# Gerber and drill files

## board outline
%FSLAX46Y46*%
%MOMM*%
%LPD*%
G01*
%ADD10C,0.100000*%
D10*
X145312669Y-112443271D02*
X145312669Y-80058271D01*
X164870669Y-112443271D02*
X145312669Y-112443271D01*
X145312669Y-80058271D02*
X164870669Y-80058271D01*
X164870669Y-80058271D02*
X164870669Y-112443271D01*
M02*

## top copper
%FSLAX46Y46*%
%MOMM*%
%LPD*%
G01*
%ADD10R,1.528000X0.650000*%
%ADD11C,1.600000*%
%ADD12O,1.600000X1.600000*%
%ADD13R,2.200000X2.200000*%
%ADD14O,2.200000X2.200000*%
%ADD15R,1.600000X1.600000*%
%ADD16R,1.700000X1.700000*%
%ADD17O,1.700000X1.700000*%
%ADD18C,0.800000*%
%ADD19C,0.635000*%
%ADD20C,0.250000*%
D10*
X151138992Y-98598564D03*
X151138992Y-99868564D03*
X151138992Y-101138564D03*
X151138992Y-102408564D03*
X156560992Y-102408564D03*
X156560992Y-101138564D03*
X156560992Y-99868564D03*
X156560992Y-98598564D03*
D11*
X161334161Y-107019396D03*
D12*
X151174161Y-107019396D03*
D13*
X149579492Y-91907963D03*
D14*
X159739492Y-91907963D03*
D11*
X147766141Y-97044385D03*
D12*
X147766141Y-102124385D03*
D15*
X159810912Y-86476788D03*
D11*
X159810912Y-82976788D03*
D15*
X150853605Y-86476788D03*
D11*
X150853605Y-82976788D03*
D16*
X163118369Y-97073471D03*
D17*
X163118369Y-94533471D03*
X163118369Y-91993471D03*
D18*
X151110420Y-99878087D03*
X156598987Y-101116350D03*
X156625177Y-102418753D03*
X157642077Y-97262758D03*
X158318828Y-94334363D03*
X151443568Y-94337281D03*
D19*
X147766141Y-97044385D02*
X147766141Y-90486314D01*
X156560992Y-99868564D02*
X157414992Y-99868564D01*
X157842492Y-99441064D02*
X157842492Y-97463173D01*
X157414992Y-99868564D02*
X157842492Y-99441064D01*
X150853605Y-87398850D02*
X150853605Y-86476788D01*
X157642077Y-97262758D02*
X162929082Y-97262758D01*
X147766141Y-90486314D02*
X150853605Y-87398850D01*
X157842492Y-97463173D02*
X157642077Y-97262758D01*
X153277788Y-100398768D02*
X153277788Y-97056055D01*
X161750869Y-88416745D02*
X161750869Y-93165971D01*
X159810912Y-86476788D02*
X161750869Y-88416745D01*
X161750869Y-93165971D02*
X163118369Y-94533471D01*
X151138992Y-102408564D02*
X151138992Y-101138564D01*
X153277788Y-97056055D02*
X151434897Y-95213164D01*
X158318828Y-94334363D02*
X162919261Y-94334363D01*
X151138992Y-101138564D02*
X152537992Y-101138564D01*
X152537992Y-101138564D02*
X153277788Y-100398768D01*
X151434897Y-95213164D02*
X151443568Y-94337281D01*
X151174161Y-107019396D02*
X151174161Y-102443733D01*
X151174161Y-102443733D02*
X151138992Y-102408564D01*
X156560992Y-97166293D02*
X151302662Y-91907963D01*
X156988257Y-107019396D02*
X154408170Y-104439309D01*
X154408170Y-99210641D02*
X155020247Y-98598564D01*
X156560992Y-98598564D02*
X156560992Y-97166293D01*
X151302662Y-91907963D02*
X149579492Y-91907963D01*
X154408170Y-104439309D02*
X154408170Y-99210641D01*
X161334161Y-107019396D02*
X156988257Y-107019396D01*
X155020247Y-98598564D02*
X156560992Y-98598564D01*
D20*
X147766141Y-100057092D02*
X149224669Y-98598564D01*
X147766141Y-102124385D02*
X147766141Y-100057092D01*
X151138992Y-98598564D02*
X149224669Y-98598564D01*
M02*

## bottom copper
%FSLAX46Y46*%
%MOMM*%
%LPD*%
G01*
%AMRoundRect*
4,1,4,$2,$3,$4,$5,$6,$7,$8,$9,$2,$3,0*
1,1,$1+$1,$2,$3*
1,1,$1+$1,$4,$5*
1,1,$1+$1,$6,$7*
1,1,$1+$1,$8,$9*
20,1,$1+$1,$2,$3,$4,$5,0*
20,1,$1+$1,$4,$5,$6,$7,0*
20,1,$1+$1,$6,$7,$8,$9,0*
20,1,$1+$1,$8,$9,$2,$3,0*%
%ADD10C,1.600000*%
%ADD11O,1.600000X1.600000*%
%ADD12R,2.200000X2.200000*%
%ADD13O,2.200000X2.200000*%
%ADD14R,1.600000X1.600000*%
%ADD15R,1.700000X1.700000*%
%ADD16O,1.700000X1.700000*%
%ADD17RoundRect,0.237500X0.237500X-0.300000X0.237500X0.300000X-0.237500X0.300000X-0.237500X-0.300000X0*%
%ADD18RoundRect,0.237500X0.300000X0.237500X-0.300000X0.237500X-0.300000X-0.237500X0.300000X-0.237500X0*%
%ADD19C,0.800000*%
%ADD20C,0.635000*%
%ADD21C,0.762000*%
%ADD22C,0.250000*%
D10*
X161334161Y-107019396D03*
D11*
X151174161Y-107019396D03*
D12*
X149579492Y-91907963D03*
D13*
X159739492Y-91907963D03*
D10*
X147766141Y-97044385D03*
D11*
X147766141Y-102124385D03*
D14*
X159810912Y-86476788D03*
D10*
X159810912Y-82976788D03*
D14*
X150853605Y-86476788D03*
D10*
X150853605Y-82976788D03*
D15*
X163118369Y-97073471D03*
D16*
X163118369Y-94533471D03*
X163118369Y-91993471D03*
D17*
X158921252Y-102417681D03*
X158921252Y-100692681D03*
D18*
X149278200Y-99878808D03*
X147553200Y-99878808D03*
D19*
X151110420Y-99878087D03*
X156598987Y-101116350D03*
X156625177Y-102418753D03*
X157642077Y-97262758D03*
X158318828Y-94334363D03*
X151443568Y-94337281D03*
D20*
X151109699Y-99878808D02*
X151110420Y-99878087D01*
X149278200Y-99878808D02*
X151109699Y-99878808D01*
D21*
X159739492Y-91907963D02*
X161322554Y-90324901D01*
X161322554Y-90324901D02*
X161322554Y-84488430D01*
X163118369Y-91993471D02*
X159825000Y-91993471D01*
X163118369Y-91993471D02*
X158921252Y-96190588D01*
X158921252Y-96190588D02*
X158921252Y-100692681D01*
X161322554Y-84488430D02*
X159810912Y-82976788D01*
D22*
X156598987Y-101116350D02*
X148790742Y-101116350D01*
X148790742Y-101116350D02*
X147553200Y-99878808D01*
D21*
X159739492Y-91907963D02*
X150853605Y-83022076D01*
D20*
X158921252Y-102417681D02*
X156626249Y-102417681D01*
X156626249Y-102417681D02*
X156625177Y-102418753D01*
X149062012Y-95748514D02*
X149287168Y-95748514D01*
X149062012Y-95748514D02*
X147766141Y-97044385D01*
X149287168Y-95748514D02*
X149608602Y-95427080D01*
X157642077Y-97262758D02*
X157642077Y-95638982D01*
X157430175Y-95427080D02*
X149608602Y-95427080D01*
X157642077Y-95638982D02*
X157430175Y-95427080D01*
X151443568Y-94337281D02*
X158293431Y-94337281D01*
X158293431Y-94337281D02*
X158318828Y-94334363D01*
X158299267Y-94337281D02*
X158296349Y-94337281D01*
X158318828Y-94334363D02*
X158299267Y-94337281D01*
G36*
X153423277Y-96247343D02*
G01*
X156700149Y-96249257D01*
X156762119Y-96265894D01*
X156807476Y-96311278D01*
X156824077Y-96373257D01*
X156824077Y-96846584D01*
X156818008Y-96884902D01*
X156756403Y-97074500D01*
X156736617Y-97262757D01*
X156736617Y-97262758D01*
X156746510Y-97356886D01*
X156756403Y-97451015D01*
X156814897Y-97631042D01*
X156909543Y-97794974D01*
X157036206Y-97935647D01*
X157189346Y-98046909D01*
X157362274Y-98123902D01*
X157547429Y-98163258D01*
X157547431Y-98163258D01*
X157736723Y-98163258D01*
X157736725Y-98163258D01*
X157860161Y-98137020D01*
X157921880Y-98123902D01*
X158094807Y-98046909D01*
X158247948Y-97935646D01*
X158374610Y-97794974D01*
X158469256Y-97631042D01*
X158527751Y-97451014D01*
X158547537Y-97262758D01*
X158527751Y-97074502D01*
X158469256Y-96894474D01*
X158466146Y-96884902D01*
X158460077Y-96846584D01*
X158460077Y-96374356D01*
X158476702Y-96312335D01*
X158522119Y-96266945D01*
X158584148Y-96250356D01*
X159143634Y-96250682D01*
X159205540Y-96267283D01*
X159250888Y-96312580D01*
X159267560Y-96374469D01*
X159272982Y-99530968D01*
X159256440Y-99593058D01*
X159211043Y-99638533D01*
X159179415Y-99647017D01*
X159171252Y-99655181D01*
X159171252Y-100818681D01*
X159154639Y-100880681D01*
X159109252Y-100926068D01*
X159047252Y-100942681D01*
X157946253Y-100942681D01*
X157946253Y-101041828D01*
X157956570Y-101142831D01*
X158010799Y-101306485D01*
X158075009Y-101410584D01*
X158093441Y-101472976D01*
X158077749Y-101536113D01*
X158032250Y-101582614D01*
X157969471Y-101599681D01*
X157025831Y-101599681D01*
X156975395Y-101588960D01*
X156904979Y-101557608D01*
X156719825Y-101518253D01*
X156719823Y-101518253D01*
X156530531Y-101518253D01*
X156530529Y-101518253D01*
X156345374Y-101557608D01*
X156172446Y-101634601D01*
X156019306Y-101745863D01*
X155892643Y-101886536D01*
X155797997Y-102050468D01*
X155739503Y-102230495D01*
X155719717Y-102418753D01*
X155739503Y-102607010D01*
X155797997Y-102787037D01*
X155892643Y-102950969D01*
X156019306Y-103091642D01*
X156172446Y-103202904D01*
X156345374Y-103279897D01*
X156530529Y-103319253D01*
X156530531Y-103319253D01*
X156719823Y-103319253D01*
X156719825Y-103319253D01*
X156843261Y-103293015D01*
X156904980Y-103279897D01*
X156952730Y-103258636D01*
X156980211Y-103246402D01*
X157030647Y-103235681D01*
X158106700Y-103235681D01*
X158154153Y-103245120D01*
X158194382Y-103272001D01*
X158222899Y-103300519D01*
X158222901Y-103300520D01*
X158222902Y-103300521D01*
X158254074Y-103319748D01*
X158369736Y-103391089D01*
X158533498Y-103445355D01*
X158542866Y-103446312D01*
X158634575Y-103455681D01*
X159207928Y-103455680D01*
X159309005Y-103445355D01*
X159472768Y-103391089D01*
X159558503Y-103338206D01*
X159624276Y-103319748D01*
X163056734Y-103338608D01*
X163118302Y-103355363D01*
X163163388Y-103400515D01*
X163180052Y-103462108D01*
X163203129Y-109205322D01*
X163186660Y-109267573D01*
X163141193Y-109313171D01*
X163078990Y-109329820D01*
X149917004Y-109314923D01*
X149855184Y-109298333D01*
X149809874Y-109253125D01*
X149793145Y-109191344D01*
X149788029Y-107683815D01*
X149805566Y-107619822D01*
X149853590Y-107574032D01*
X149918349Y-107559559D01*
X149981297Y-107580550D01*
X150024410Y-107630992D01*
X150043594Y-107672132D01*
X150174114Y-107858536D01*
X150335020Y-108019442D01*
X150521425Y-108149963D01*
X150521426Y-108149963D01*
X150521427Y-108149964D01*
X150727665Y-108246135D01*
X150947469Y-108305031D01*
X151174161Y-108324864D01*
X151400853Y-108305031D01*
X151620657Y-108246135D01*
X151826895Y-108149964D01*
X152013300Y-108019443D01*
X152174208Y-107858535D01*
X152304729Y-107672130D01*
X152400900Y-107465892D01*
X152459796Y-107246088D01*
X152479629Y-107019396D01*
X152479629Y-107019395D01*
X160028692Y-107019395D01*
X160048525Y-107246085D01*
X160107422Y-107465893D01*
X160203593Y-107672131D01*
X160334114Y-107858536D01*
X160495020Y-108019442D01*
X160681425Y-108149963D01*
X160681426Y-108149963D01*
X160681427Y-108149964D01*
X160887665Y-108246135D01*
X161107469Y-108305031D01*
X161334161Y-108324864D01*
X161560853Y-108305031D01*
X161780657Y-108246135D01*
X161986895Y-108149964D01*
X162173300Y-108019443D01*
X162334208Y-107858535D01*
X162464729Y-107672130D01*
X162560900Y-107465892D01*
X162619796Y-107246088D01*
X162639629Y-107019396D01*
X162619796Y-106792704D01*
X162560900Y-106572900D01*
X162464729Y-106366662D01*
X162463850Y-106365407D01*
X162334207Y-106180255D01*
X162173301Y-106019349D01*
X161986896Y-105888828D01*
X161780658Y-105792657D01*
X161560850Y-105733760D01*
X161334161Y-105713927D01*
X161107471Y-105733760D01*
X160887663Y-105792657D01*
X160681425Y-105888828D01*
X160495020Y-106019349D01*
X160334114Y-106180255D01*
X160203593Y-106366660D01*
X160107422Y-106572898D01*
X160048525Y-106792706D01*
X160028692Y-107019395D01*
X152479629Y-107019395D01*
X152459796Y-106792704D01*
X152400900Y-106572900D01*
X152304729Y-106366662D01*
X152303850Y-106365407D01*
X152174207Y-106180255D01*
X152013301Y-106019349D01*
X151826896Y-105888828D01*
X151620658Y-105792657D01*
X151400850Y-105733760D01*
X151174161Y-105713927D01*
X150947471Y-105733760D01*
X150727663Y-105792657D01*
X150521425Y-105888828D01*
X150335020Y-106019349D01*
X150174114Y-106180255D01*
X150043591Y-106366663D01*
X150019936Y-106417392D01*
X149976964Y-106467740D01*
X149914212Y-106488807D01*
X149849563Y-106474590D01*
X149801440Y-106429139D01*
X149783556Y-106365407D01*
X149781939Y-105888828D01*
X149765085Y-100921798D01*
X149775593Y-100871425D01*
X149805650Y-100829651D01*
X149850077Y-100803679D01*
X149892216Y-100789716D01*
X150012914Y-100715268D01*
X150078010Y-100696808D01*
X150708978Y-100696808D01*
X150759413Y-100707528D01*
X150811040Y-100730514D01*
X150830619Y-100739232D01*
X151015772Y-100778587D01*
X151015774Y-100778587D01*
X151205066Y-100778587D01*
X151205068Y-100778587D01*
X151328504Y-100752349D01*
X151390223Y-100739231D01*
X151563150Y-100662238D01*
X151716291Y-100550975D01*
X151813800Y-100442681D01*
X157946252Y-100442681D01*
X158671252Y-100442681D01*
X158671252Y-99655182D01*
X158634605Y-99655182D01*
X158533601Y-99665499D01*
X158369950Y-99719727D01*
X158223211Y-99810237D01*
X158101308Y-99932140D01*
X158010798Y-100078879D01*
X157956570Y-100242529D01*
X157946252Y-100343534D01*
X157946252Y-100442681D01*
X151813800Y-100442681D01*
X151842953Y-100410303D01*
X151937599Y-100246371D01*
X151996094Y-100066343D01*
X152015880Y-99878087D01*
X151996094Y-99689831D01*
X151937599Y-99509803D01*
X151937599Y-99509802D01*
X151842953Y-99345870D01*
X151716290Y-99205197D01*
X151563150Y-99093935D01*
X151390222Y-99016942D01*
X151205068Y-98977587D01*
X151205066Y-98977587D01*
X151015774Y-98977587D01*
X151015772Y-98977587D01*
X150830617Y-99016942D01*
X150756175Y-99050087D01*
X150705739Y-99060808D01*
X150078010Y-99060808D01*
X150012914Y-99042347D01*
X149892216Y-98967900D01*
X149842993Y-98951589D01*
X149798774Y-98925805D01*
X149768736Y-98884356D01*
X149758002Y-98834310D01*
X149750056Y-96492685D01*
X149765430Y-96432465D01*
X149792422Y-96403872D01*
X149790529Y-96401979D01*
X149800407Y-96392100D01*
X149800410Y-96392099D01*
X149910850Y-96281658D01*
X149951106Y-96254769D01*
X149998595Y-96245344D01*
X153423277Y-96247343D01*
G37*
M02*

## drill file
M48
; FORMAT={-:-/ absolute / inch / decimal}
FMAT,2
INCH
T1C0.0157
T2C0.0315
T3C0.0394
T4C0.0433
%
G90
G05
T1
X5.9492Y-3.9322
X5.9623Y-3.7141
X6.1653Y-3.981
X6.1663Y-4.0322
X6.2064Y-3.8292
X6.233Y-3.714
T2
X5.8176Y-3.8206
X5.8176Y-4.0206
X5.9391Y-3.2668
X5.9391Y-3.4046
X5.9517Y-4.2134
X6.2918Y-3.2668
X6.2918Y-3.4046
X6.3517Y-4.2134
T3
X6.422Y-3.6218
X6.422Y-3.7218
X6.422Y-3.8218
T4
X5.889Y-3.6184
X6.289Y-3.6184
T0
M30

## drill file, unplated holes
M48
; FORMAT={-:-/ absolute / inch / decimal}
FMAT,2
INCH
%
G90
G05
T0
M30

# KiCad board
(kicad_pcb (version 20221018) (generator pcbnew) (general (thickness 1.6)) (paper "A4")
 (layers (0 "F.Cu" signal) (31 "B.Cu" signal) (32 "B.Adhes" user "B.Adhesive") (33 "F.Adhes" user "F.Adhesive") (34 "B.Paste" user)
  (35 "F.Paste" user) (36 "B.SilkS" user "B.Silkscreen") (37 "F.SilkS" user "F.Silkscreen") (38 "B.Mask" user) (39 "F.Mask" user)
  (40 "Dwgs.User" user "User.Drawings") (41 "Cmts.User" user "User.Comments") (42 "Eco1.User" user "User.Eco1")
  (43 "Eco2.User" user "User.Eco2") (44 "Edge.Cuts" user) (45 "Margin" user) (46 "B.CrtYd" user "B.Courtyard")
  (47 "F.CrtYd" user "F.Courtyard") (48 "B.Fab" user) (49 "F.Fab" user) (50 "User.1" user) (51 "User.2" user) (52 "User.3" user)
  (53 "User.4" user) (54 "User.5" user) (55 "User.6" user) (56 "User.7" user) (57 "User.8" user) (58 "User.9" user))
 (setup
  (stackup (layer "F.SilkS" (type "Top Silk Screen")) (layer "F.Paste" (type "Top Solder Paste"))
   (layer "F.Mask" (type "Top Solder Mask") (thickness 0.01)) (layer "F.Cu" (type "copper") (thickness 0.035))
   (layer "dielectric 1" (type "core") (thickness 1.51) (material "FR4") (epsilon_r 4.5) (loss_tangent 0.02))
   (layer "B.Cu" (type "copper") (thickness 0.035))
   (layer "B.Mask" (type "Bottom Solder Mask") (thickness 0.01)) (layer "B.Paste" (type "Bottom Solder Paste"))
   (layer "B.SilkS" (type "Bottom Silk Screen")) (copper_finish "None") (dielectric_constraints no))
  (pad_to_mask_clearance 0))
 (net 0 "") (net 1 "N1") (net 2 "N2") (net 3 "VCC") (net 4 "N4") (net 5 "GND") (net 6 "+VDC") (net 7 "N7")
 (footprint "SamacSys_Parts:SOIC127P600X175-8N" (layer "F.Cu") (at 153.849992 100.503564)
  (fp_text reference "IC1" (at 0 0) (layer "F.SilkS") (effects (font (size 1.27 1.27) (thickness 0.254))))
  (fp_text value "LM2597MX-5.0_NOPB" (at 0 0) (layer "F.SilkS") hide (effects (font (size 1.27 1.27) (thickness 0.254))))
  (pad "1" smd rect (at -2.711 -1.905 90) (size 0.65 1.528) (layers "F.Cu" "F.Paste" "F.Mask") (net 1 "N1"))
  (pad "2" smd rect (at -2.711 -0.635 90) (size 0.65 1.528) (layers "F.Cu" "F.Paste" "F.Mask") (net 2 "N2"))
  (pad "3" smd rect (at -2.711 0.635 90) (size 0.65 1.528) (layers "F.Cu" "F.Paste" "F.Mask") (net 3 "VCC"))
  (pad "4" smd rect (at -2.711 1.905 90) (size 0.65 1.528) (layers "F.Cu" "F.Paste" "F.Mask") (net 3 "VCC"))
  (pad "5" smd rect (at 2.711 1.905 90) (size 0.65 1.528) (layers "F.Cu" "F.Paste" "F.Mask") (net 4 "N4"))
  (pad "6" smd rect (at 2.711 0.635 90) (size 0.65 1.528) (layers "F.Cu" "F.Paste" "F.Mask") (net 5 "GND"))
  (pad "7" smd rect (at 2.711 -0.635 90) (size 0.65 1.528) (layers "F.Cu" "F.Paste" "F.Mask") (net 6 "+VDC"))
  (pad "8" smd rect (at 2.711 -1.905 90) (size 0.65 1.528) (layers "F.Cu" "F.Paste" "F.Mask") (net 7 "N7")))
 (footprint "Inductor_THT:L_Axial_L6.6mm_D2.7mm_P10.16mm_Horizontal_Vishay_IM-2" (layer "F.Cu") (at 161.334161 107.019396 180)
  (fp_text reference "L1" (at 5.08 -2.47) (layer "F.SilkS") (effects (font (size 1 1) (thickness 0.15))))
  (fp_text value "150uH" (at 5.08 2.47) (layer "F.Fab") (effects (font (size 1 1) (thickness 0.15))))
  (pad "1" thru_hole circle (at 0 0 180) (size 1.6 1.6) (drill 0.8) (layers "*.Cu" "*.Mask") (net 7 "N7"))
  (pad "2" thru_hole oval (at 10.16 0 180) (size 1.6 1.6) (drill 0.8) (layers "*.Cu" "*.Mask") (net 3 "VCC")))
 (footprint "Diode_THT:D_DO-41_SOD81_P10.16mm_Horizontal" (layer "F.Cu") (at 149.579492 91.907963)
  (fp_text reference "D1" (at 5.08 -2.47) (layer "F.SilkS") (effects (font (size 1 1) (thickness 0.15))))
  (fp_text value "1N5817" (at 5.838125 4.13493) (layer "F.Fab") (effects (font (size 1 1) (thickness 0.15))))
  (pad "1" thru_hole rect (at 0 0) (size 2.2 2.2) (drill 1.1) (layers "*.Cu" "*.Mask") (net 7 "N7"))
  (pad "2" thru_hole oval (at 10.16 0) (size 2.2 2.2) (drill 1.1) (layers "*.Cu" "*.Mask") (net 5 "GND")))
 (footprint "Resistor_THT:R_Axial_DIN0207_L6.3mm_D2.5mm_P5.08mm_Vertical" (layer "F.Cu") (at 147.766141 97.044385 -90)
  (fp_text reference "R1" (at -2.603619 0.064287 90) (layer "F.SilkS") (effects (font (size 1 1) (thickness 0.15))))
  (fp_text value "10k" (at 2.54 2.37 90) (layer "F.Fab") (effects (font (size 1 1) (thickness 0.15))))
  (pad "1" thru_hole circle (at 0 0 270) (size 1.6 1.6) (drill 0.8) (layers "*.Cu" "*.Mask") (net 6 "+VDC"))
  (pad "2" thru_hole oval (at 5.08 0 270) (size 1.6 1.6) (drill 0.8) (layers "*.Cu" "*.Mask") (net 1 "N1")))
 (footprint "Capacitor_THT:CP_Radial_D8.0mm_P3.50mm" (layer "F.Cu") (at 159.810912 86.476788 90)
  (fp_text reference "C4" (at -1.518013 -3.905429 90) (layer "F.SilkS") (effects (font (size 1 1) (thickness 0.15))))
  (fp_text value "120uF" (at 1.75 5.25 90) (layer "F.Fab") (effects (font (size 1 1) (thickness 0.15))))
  (pad "1" thru_hole rect (at 0 0 90) (size 1.6 1.6) (drill 0.8) (layers "*.Cu" "*.Mask") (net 3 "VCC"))
  (pad "2" thru_hole circle (at 3.5 0 90) (size 1.6 1.6) (drill 0.8) (layers "*.Cu" "*.Mask") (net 5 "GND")))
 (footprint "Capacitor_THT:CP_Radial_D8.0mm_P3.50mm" (layer "F.Cu") (at 150.853605 86.476788 90)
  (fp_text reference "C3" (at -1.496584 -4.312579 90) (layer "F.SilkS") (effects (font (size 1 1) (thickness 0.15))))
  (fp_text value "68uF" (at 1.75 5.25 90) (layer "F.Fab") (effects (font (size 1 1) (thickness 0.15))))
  (pad "1" thru_hole rect (at 0 0 90) (size 1.6 1.6) (drill 0.8) (layers "*.Cu" "*.Mask") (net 6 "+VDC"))
  (pad "2" thru_hole circle (at 3.5 0 90) (size 1.6 1.6) (drill 0.8) (layers "*.Cu" "*.Mask") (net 5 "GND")))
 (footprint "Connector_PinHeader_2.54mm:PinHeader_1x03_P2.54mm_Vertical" (layer "F.Cu") (at 163.118369 97.073471 180)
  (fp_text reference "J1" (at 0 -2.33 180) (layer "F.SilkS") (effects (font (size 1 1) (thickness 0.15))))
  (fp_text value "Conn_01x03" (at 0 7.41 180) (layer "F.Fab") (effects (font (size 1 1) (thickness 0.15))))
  (pad "1" thru_hole rect (at 0 0 180) (size 1.7 1.7) (drill 1) (layers "*.Cu" "*.Mask") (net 6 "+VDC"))
  (pad "2" thru_hole oval (at 0 2.54 180) (size 1.7 1.7) (drill 1) (layers "*.Cu" "*.Mask") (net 3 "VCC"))
  (pad "3" thru_hole oval (at 0 5.08 180) (size 1.7 1.7) (drill 1) (layers "*.Cu" "*.Mask") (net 5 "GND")))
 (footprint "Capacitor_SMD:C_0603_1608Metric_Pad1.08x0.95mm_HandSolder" (layer "B.Cu") (at 158.921252 101.555181 90)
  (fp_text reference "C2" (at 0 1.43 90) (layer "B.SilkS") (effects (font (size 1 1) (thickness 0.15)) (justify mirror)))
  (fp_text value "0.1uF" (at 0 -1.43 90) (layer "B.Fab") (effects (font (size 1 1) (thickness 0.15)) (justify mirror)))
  (pad "1" smd roundrect (at -0.8625 0 90) (size 1.075 0.95) (layers "B.Cu" "B.Paste" "B.Mask") (roundrect_rratio 0.25) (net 4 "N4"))
  (pad "2" smd roundrect (at 0.8625 0 90) (size 1.075 0.95) (layers "B.Cu" "B.Paste" "B.Mask") (roundrect_rratio 0.25) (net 5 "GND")))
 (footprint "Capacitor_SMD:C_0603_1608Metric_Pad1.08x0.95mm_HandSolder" (layer "B.Cu") (at 148.4157 99.878808 180)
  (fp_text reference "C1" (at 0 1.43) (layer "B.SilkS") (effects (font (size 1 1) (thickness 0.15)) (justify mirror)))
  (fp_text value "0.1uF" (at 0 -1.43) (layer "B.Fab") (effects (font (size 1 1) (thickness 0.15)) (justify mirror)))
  (pad "1" smd roundrect (at -0.8625 0 180) (size 1.075 0.95) (layers "B.Cu" "B.Paste" "B.Mask") (roundrect_rratio 0.25) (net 2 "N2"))
  (pad "2" smd roundrect (at 0.8625 0 180) (size 1.075 0.95) (layers "B.Cu" "B.Paste" "B.Mask") (roundrect_rratio 0.25) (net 5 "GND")))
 (gr_line (start 145.312669 112.443271) (end 145.312669 80.058271) (stroke (width 0.1) (type solid)) (layer "Edge.Cuts"))
 (gr_line (start 164.870669 112.443271) (end 145.312669 112.443271) (stroke (width 0.1) (type default)) (layer "Edge.Cuts"))
 (gr_line (start 145.312669 80.058271) (end 164.870669 80.058271) (stroke (width 0.1) (type solid)) (layer "Edge.Cuts"))
 (gr_line (start 164.870669 80.058271) (end 164.870669 112.443271) (stroke (width 0.1) (type default)) (layer "Edge.Cuts"))
 (via (at 151.11042 99.878087) (size 0.8) (drill 0.4) (layers "F.Cu" "B.Cu") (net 2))
 (segment (start 151.109699 99.878808) (end 151.11042 99.878087) (width 0.635) (layer "B.Cu") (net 2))
 (segment (start 149.2782 99.878808) (end 151.109699 99.878808) (width 0.635) (layer "B.Cu") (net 2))
 (via (at 156.598987 101.11635) (size 0.8) (drill 0.4) (layers "F.Cu" "B.Cu") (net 5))
 (segment (start 159.739492 91.907963) (end 161.322554 90.324901) (width 0.762) (layer "B.Cu") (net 5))
 (segment (start 161.322554 90.324901) (end 161.322554 84.48843) (width 0.762) (layer "B.Cu") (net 5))
 (segment (start 163.118369 91.993471) (end 159.825 91.993471) (width 0.762) (layer "B.Cu") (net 5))
 (segment (start 163.118369 91.993471) (end 158.921252 96.190588) (width 0.762) (layer "B.Cu") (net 5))
 (segment (start 158.921252 96.190588) (end 158.921252 100.692681) (width 0.762) (layer "B.Cu") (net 5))
 (segment (start 161.322554 84.48843) (end 159.810912 82.976788) (width 0.762) (layer "B.Cu") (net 5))
 (segment (start 156.598987 101.11635) (end 148.790742 101.11635) (width 0.25) (layer "B.Cu") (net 5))
 (segment (start 148.790742 101.11635) (end 147.5532 99.878808) (width 0.25) (layer "B.Cu") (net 5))
 (segment (start 159.739492 91.907963) (end 150.853605 83.022076) (width 0.762) (layer "B.Cu") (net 5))
 (via (at 156.625177 102.418753) (size 0.8) (drill 0.4) (layers "F.Cu" "B.Cu") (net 4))
 (segment (start 158.921252 102.417681) (end 156.626249 102.417681) (width 0.635) (layer "B.Cu") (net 4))
 (segment (start 156.626249 102.417681) (end 156.625177 102.418753) (width 0.635) (layer "B.Cu") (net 4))
 (segment (start 147.766141 97.044385) (end 147.766141 90.486314) (width 0.635) (layer "F.Cu") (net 6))
 (segment (start 156.560992 99.868564) (end 157.414992 99.868564) (width 0.635) (layer "F.Cu") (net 6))
 (segment (start 157.842492 99.441064) (end 157.842492 97.463173) (width 0.635) (layer "F.Cu") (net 6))
 (segment (start 157.414992 99.868564) (end 157.842492 99.441064) (width 0.635) (layer "F.Cu") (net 6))
 (segment (start 150.853605 87.39885) (end 150.853605 86.476788) (width 0.635) (layer "F.Cu") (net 6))
 (segment (start 157.642077 97.262758) (end 162.929082 97.262758) (width 0.635) (layer "F.Cu") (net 6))
 (segment (start 147.766141 90.486314) (end 150.853605 87.39885) (width 0.635) (layer "F.Cu") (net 6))
 (segment (start 157.842492 97.463173) (end 157.642077 97.262758) (width 0.635) (layer "F.Cu") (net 6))
 (via (at 157.642077 97.262758) (size 0.8) (drill 0.4) (layers "F.Cu" "B.Cu") (free) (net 6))
 (segment (start 149.062012 95.748514) (end 149.287168 95.748514) (width 0.635) (layer "B.Cu") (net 6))
 (segment (start 149.062012 95.748514) (end 147.766141 97.044385) (width 0.635) (layer "B.Cu") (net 6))
 (segment (start 149.287168 95.748514) (end 149.608602 95.42708) (width 0.635) (layer "B.Cu") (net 6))
 (segment (start 157.642077 97.262758) (end 157.642077 95.638982) (width 0.635) (layer "B.Cu") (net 6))
 (segment (start 157.430175 95.42708) (end 149.608602 95.42708) (width 0.635) (layer "B.Cu") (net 6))
 (segment (start 157.642077 95.638982) (end 157.430175 95.42708) (width 0.635) (layer "B.Cu") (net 6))
 (segment (start 153.277788 100.398768) (end 153.277788 97.056055) (width 0.635) (layer "F.Cu") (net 3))
 (segment (start 161.750869 88.416745) (end 161.750869 93.165971) (width 0.635) (layer "F.Cu") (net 3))
 (segment (start 159.810912 86.476788) (end 161.750869 88.416745) (width 0.635) (layer "F.Cu") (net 3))
 (segment (start 161.750869 93.165971) (end 163.118369 94.533471) (width 0.635) (layer "F.Cu") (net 3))
 (segment (start 151.138992 102.408564) (end 151.138992 101.138564) (width 0.635) (layer "F.Cu") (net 3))
 (segment (start 153.277788 97.056055) (end 151.434897 95.213164) (width 0.635) (layer "F.Cu") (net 3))
 (segment (start 158.318828 94.334363) (end 162.919261 94.334363) (width 0.635) (layer "F.Cu") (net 3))
 (segment (start 151.138992 101.138564) (end 152.537992 101.138564) (width 0.635) (layer "F.Cu") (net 3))
 (segment (start 152.537992 101.138564) (end 153.277788 100.398768) (width 0.635) (layer "F.Cu") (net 3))
 (segment (start 151.434897 95.213164) (end 151.443568 94.337281) (width 0.635) (layer "F.Cu") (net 3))
 (segment (start 151.174161 107.019396) (end 151.174161 102.443733) (width 0.635) (layer "F.Cu") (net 3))
 (segment (start 151.174161 102.443733) (end 151.138992 102.408564) (width 0.635) (layer "F.Cu") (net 3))
 (via (at 158.318828 94.334363) (size 0.8) (drill 0.4) (layers "F.Cu" "B.Cu") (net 3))
 (via (at 151.443568 94.337281) (size 0.8) (drill 0.4) (layers "F.Cu" "B.Cu") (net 3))
 (segment (start 151.443568 94.337281) (end 158.293431 94.337281) (width 0.635) (layer "B.Cu") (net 3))
 (segment (start 158.293431 94.337281) (end 158.318828 94.334363) (width 0.635) (layer "B.Cu") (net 3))
 (segment (start 158.299267 94.337281) (end 158.296349 94.337281) (width 0.635) (layer "B.Cu") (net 3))
 (segment (start 158.318828 94.334363) (end 158.299267 94.337281) (width 0.635) (layer "B.Cu") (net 3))
 (segment (start 156.560992 97.166293) (end 151.302662 91.907963) (width 0.635) (layer "F.Cu") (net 7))
 (segment (start 156.988257 107.019396) (end 154.40817 104.439309) (width 0.635) (layer "F.Cu") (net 7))
 (segment (start 154.40817 99.210641) (end 155.020247 98.598564) (width 0.635) (layer "F.Cu") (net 7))
 (segment (start 156.560992 98.598564) (end 156.560992 97.166293) (width 0.635) (layer "F.Cu") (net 7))
 (segment (start 151.302662 91.907963) (end 149.579492 91.907963) (width 0.635) (layer "F.Cu") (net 7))
 (segment (start 154.40817 104.439309) (end 154.40817 99.210641) (width 0.635) (layer "F.Cu") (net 7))
 (segment (start 161.334161 107.019396) (end 156.988257 107.019396) (width 0.635) (layer "F.Cu") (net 7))
 (segment (start 155.020247 98.598564) (end 156.560992 98.598564) (width 0.635) (layer "F.Cu") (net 7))
 (segment (start 147.766141 100.057092) (end 149.224669 98.598564) (width 0.25) (layer "F.Cu") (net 1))
 (segment (start 147.766141 102.124385) (end 147.766141 100.057092) (width 0.25) (layer "F.Cu") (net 1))
 (segment (start 151.138992 98.598564) (end 149.224669 98.598564) (width 0.25) (layer "F.Cu") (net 1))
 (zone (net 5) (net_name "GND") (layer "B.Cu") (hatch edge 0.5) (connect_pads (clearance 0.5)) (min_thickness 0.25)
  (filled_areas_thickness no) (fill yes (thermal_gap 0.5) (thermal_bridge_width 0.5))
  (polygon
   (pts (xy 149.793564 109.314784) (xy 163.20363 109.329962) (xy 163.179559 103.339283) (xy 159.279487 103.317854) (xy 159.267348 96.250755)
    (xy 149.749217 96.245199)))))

